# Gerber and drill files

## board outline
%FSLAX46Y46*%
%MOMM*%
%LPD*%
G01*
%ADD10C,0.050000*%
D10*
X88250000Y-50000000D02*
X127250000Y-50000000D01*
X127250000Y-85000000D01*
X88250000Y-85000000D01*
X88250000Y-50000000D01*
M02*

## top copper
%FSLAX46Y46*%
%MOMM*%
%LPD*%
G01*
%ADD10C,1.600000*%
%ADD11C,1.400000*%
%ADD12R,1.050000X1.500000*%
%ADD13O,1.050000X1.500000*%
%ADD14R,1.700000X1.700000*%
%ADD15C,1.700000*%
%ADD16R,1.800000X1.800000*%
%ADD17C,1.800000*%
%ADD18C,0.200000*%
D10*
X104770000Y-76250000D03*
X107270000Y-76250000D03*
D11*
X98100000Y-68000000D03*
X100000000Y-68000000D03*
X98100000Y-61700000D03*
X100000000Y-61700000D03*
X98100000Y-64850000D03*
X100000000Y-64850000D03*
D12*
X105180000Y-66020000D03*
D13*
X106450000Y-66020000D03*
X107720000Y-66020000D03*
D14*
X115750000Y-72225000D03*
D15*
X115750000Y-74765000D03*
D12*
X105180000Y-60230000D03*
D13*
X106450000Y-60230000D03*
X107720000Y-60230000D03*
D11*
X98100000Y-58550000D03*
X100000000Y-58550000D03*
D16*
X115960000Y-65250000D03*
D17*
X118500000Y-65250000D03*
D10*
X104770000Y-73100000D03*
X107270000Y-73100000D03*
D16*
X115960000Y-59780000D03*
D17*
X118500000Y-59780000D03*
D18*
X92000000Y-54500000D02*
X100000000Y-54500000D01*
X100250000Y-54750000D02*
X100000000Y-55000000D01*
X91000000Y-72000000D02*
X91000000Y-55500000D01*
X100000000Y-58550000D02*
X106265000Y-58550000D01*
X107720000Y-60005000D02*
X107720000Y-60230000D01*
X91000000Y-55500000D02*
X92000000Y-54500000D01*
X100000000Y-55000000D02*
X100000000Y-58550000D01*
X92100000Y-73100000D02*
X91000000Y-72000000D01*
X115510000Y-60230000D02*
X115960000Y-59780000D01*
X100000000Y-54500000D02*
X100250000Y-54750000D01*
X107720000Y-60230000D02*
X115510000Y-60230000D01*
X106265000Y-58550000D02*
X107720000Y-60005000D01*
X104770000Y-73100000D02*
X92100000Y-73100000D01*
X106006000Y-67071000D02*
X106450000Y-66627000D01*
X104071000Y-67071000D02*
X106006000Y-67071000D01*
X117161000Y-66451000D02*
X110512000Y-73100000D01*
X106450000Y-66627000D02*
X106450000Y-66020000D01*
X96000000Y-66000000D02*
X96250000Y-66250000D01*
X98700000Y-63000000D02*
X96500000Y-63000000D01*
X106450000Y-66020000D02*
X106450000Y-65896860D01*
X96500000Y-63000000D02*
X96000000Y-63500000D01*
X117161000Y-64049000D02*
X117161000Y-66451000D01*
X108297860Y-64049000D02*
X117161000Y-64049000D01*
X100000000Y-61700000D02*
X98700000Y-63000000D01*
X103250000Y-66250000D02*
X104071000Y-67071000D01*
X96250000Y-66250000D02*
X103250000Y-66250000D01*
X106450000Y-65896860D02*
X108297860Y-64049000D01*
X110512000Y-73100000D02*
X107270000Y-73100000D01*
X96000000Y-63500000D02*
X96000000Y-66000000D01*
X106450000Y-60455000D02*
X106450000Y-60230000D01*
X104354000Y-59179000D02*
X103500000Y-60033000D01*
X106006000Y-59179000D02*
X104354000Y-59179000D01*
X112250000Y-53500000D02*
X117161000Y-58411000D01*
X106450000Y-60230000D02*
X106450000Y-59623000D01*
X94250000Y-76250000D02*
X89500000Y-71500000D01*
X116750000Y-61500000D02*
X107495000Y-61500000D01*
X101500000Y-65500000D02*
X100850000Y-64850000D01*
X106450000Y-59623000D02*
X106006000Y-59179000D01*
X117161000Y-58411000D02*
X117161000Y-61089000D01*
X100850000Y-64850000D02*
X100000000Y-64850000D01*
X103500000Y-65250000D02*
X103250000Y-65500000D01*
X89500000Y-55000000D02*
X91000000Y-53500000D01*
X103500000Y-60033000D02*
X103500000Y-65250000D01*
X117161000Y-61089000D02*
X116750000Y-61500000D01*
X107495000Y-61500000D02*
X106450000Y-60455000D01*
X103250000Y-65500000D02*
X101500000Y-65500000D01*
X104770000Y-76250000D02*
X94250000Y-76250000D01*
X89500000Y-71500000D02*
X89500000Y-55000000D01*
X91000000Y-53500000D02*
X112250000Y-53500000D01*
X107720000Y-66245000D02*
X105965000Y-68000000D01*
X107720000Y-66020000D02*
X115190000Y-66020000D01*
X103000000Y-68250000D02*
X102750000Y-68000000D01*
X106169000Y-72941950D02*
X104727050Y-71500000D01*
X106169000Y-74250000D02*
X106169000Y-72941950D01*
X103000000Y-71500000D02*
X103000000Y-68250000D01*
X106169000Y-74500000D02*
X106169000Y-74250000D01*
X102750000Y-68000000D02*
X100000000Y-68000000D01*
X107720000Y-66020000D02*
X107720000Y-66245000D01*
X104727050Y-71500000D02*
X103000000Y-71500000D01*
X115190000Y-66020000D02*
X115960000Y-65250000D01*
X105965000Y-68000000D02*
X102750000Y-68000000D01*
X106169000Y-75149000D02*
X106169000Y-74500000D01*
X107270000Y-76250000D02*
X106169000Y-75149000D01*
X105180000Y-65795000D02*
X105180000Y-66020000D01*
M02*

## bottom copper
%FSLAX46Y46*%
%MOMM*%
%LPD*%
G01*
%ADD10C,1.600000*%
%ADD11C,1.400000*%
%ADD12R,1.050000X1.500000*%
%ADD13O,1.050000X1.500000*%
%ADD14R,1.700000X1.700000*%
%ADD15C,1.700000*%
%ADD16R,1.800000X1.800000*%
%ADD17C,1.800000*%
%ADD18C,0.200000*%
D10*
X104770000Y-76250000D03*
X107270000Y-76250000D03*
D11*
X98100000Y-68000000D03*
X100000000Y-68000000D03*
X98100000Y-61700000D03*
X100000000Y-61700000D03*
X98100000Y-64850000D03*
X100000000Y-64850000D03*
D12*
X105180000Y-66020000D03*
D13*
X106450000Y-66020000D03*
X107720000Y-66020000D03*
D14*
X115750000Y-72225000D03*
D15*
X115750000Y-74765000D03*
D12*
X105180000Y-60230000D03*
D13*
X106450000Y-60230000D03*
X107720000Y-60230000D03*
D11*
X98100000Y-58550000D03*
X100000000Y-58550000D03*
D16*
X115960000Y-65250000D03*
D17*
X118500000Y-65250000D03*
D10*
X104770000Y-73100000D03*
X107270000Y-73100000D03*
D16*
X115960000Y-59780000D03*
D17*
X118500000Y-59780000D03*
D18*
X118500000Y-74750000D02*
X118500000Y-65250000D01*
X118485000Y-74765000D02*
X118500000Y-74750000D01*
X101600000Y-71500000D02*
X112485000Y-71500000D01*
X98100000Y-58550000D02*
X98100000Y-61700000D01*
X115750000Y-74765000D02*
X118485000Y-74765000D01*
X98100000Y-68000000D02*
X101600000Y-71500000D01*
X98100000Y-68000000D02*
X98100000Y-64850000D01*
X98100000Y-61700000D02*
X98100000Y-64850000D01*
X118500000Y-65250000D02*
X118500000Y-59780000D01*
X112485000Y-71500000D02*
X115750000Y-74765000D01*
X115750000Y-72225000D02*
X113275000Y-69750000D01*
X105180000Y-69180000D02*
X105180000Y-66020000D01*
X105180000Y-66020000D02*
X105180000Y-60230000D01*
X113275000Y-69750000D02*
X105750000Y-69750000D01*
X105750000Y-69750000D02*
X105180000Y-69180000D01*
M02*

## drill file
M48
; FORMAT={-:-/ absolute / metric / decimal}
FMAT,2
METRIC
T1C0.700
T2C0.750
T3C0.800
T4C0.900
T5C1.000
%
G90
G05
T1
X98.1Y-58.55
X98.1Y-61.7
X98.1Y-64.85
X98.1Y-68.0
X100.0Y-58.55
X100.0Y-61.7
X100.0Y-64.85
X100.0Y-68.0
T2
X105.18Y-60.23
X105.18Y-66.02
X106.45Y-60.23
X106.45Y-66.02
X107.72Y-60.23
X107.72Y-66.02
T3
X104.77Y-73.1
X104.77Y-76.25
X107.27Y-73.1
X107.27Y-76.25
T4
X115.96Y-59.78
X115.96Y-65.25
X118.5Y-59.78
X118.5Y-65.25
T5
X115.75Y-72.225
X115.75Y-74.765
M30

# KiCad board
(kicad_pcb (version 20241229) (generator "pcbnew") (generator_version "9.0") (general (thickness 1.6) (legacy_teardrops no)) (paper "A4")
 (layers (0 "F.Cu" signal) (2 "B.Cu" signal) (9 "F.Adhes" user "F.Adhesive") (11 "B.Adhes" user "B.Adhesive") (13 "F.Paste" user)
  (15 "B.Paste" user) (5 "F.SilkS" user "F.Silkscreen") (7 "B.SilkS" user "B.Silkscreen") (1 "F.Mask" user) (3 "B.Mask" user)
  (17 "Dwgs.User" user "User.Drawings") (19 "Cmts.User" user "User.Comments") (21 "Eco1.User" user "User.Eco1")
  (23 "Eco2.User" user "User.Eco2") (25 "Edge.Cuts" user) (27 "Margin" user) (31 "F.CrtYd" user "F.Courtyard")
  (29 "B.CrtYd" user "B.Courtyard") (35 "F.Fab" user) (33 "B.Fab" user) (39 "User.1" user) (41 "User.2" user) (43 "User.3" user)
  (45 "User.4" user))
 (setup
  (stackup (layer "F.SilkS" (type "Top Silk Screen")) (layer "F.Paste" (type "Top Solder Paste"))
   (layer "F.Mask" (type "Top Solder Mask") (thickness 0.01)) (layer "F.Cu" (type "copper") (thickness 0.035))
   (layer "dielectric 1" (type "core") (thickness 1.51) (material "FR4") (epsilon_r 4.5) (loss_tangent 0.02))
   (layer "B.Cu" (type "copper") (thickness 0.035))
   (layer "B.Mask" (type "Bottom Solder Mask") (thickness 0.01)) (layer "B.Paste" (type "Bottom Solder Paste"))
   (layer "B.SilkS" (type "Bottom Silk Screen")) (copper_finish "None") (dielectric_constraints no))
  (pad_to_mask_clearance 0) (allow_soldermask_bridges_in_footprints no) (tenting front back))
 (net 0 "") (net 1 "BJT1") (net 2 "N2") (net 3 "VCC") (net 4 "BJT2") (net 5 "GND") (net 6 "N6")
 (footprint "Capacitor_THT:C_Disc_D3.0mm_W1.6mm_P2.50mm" (layer "F.Cu") (at 104.77 76.25)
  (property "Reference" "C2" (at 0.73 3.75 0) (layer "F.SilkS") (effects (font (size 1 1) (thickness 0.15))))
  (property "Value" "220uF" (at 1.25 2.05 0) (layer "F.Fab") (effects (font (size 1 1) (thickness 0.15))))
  (pad "1" thru_hole circle (at 0 0) (size 1.6 1.6) (drill 0.8) (layers "*.Cu" "*.Mask") (remove_unused_layers no) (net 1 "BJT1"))
  (pad "2" thru_hole circle (at 2.5 0) (size 1.6 1.6) (drill 0.8) (layers "*.Cu" "*.Mask") (remove_unused_layers no) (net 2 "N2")))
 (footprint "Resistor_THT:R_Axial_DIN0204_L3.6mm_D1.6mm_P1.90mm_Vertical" (layer "F.Cu") (at 98.1 68)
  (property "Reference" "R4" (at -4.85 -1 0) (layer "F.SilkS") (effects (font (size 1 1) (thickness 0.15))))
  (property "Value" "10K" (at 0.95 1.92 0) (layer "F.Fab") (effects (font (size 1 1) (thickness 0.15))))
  (pad "1" thru_hole circle (at 0 0) (size 1.4 1.4) (drill 0.7) (layers "*.Cu" "*.Mask") (remove_unused_layers no) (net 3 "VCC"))
  (pad "2" thru_hole circle (at 1.9 0) (size 1.4 1.4) (drill 0.7) (layers "*.Cu" "*.Mask") (remove_unused_layers no) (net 2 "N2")))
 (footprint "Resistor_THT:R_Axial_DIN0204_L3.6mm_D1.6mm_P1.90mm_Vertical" (layer "F.Cu") (at 98.1 61.7)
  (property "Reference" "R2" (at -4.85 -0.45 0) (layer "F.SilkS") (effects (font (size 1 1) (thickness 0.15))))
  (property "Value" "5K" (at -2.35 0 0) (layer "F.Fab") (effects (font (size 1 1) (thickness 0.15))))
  (pad "1" thru_hole circle (at 0 0) (size 1.4 1.4) (drill 0.7) (layers "*.Cu" "*.Mask") (remove_unused_layers no) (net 3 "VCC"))
  (pad "2" thru_hole circle (at 1.9 0) (size 1.4 1.4) (drill 0.7) (layers "*.Cu" "*.Mask") (remove_unused_layers no) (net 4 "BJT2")))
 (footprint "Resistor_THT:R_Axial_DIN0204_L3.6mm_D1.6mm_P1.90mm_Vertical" (layer "F.Cu") (at 98.1 64.85)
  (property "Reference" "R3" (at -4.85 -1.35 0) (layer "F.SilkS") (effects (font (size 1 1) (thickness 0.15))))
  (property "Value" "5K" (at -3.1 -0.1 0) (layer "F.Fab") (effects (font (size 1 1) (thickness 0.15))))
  (pad "1" thru_hole circle (at 0 0) (size 1.4 1.4) (drill 0.7) (layers "*.Cu" "*.Mask") (remove_unused_layers no) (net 3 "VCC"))
  (pad "2" thru_hole circle (at 1.9 0) (size 1.4 1.4) (drill 0.7) (layers "*.Cu" "*.Mask") (remove_unused_layers no) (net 1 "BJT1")))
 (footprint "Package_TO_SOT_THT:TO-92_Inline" (layer "F.Cu") (at 105.18 66.02)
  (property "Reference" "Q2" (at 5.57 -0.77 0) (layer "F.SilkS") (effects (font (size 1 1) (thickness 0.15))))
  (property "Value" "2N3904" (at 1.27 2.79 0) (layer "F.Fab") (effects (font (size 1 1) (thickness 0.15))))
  (pad "1" thru_hole rect (at 0 0) (size 1.05 1.5) (drill 0.75) (layers "*.Cu" "*.Mask") (remove_unused_layers no) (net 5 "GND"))
  (pad "2" thru_hole oval (at 1.27 0) (size 1.05 1.5) (drill 0.75) (layers "*.Cu" "*.Mask") (remove_unused_layers no) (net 4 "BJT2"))
  (pad "3" thru_hole oval (at 2.54 0) (size 1.05 1.5) (drill 0.75) (layers "*.Cu" "*.Mask") (remove_unused_layers no) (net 2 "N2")))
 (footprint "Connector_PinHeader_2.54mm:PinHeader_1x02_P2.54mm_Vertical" (layer "F.Cu") (at 115.75 72.225)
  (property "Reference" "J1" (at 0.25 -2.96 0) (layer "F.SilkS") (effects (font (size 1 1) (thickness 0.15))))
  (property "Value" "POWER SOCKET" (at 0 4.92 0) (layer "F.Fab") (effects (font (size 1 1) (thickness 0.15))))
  (pad "1" thru_hole rect (at 0 0) (size 1.7 1.7) (drill 1) (layers "*.Cu" "*.Mask") (remove_unused_layers no) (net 5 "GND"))
  (pad "2" thru_hole circle (at 0 2.54) (size 1.7 1.7) (drill 1) (layers "*.Cu" "*.Mask") (remove_unused_layers no) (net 3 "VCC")))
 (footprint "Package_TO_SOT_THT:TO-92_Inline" (layer "F.Cu") (at 105.18 60.23)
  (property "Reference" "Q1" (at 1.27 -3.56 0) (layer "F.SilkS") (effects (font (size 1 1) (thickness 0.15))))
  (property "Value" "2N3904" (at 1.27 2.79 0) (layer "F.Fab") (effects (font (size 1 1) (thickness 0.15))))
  (pad "1" thru_hole rect (at 0 0) (size 1.05 1.5) (drill 0.75) (layers "*.Cu" "*.Mask") (remove_unused_layers no) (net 5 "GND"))
  (pad "2" thru_hole oval (at 1.27 0) (size 1.05 1.5) (drill 0.75) (layers "*.Cu" "*.Mask") (remove_unused_layers no) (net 1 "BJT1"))
  (pad "3" thru_hole oval (at 2.54 0) (size 1.05 1.5) (drill 0.75) (layers "*.Cu" "*.Mask") (remove_unused_layers no) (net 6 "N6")))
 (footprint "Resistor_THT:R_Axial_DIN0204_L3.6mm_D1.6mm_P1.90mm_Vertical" (layer "F.Cu") (at 98.1 58.55)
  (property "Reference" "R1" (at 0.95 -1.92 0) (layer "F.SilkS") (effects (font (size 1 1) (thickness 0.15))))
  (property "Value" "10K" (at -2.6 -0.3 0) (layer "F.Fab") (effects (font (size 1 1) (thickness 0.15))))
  (pad "1" thru_hole circle (at 0 0) (size 1.4 1.4) (drill 0.7) (layers "*.Cu" "*.Mask") (remove_unused_layers no) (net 3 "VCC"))
  (pad "2" thru_hole circle (at 1.9 0) (size 1.4 1.4) (drill 0.7) (layers "*.Cu" "*.Mask") (remove_unused_layers no) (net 6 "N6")))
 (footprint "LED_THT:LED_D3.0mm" (layer "F.Cu") (at 115.96 65.25)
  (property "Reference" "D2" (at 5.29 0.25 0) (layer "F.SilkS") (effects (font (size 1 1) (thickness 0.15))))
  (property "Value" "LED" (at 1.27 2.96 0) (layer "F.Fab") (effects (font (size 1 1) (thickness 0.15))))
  (pad "1" thru_hole rect (at 0 0) (size 1.8 1.8) (drill 0.9) (layers "*.Cu" "*.Mask") (remove_unused_layers no) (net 2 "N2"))
  (pad "2" thru_hole circle (at 2.54 0) (size 1.8 1.8) (drill 0.9) (layers "*.Cu" "*.Mask") (remove_unused_layers no) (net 3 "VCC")))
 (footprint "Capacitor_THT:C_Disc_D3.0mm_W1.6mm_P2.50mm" (layer "F.Cu") (at 104.77 73.1)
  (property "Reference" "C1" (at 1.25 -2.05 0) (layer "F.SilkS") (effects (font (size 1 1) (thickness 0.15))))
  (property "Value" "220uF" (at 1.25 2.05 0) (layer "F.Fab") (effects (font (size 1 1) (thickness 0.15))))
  (pad "1" thru_hole circle (at 0 0) (size 1.6 1.6) (drill 0.8) (layers "*.Cu" "*.Mask") (remove_unused_layers no) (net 6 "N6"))
  (pad "2" thru_hole circle (at 2.5 0) (size 1.6 1.6) (drill 0.8) (layers "*.Cu" "*.Mask") (remove_unused_layers no) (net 4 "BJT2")))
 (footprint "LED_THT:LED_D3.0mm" (layer "F.Cu") (at 115.96 59.78)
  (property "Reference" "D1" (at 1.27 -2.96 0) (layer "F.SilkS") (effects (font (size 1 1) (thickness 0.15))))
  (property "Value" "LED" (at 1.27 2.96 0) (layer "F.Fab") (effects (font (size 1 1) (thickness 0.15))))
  (pad "1" thru_hole rect (at 0 0) (size 1.8 1.8) (drill 0.9) (layers "*.Cu" "*.Mask") (remove_unused_layers no) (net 6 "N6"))
  (pad "2" thru_hole circle (at 2.54 0) (size 1.8 1.8) (drill 0.9) (layers "*.Cu" "*.Mask") (remove_unused_layers no) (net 3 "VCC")))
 (gr_rect (start 88.25 50) (end 127.25 85) (stroke (width 0.05) (type default)) (fill no) (layer "Edge.Cuts"))
 (segment (start 118.5 74.75) (end 118.5 65.25) (width 0.2) (layer "B.Cu") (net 3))
 (segment (start 118.485 74.765) (end 118.5 74.75) (width 0.2) (layer "B.Cu") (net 3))
 (segment (start 101.6 71.5) (end 112.485 71.5) (width 0.2) (layer "B.Cu") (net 3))
 (segment (start 98.1 58.55) (end 98.1 61.7) (width 0.2) (layer "B.Cu") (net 3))
 (segment (start 115.75 74.765) (end 118.485 74.765) (width 0.2) (layer "B.Cu") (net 3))
 (segment (start 98.1 68) (end 101.6 71.5) (width 0.2) (layer "B.Cu") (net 3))
 (segment (start 98.1 68) (end 98.1 64.85) (width 0.2) (layer "B.Cu") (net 3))
 (segment (start 98.1 61.7) (end 98.1 64.85) (width 0.2) (layer "B.Cu") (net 3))
 (segment (start 118.5 65.25) (end 118.5 59.78) (width 0.2) (layer "B.Cu") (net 3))
 (segment (start 112.485 71.5) (end 115.75 74.765) (width 0.2) (layer "B.Cu") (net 3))
 (segment (start 92 54.5) (end 100 54.5) (width 0.2) (layer "F.Cu") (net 6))
 (segment (start 100.25 54.75) (end 100 55) (width 0.2) (layer "F.Cu") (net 6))
 (segment (start 91 72) (end 91 55.5) (width 0.2) (layer "F.Cu") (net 6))
 (segment (start 100 58.55) (end 106.265 58.55) (width 0.2) (layer "F.Cu") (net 6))
 (segment (start 107.72 60.005) (end 107.72 60.23) (width 0.2) (layer "F.Cu") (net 6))
 (segment (start 91 55.5) (end 92 54.5) (width 0.2) (layer "F.Cu") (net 6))
 (segment (start 100 55) (end 100 58.55) (width 0.2) (layer "F.Cu") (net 6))
 (segment (start 92.1 73.1) (end 91 72) (width 0.2) (layer "F.Cu") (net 6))
 (segment (start 115.51 60.23) (end 115.96 59.78) (width 0.2) (layer "F.Cu") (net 6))
 (segment (start 100 54.5) (end 100.25 54.75) (width 0.2) (layer "F.Cu") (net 6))
 (segment (start 107.72 60.23) (end 115.51 60.23) (width 0.2) (layer "F.Cu") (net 6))
 (segment (start 106.265 58.55) (end 107.72 60.005) (width 0.2) (layer "F.Cu") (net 6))
 (segment (start 104.77 73.1) (end 92.1 73.1) (width 0.2) (layer "F.Cu") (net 6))
 (segment (start 106.006 67.071) (end 106.45 66.627) (width 0.2) (layer "F.Cu") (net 4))
 (segment (start 104.071 67.071) (end 106.006 67.071) (width 0.2) (layer "F.Cu") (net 4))
 (segment (start 117.161 66.451) (end 110.512 73.1) (width 0.2) (layer "F.Cu") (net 4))
 (segment (start 106.45 66.627) (end 106.45 66.02) (width 0.2) (layer "F.Cu") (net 4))
 (segment (start 96 66) (end 96.25 66.25) (width 0.2) (layer "F.Cu") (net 4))
 (segment (start 98.7 63) (end 96.5 63) (width 0.2) (layer "F.Cu") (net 4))
 (segment (start 106.45 66.02) (end 106.45 65.89686) (width 0.2) (layer "F.Cu") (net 4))
 (segment (start 96.5 63) (end 96 63.5) (width 0.2) (layer "F.Cu") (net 4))
 (segment (start 117.161 64.049) (end 117.161 66.451) (width 0.2) (layer "F.Cu") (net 4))
 (segment (start 108.29786 64.049) (end 117.161 64.049) (width 0.2) (layer "F.Cu") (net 4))
 (segment (start 100 61.7) (end 98.7 63) (width 0.2) (layer "F.Cu") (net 4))
 (segment (start 103.25 66.25) (end 104.071 67.071) (width 0.2) (layer "F.Cu") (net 4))
 (segment (start 96.25 66.25) (end 103.25 66.25) (width 0.2) (layer "F.Cu") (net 4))
 (segment (start 106.45 65.89686) (end 108.29786 64.049) (width 0.2) (layer "F.Cu") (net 4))
 (segment (start 110.512 73.1) (end 107.27 73.1) (width 0.2) (layer "F.Cu") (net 4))
 (segment (start 96 63.5) (end 96 66) (width 0.2) (layer "F.Cu") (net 4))
 (segment (start 106.45 60.455) (end 106.45 60.23) (width 0.2) (layer "F.Cu") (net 1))
 (segment (start 104.354 59.179) (end 103.5 60.033) (width 0.2) (layer "F.Cu") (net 1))
 (segment (start 106.006 59.179) (end 104.354 59.179) (width 0.2) (layer "F.Cu") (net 1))
 (segment (start 112.25 53.5) (end 117.161 58.411) (width 0.2) (layer "F.Cu") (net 1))
 (segment (start 106.45 60.23) (end 106.45 59.623) (width 0.2) (layer "F.Cu") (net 1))
 (segment (start 94.25 76.25) (end 89.5 71.5) (width 0.2) (layer "F.Cu") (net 1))
 (segment (start 116.75 61.5) (end 107.495 61.5) (width 0.2) (layer "F.Cu") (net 1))
 (segment (start 101.5 65.5) (end 100.85 64.85) (width 0.2) (layer "F.Cu") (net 1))
 (segment (start 106.45 59.623) (end 106.006 59.179) (width 0.2) (layer "F.Cu") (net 1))
 (segment (start 117.161 58.411) (end 117.161 61.089) (width 0.2) (layer "F.Cu") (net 1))
 (segment (start 100.85 64.85) (end 100 64.85) (width 0.2) (layer "F.Cu") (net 1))
 (segment (start 103.5 65.25) (end 103.25 65.5) (width 0.2) (layer "F.Cu") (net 1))
 (segment (start 89.5 55) (end 91 53.5) (width 0.2) (layer "F.Cu") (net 1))
 (segment (start 103.5 60.033) (end 103.5 65.25) (width 0.2) (layer "F.Cu") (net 1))
 (segment (start 117.161 61.089) (end 116.75 61.5) (width 0.2) (layer "F.Cu") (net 1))
 (segment (start 107.495 61.5) (end 106.45 60.455) (width 0.2) (layer "F.Cu") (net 1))
 (segment (start 103.25 65.5) (end 101.5 65.5) (width 0.2) (layer "F.Cu") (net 1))
 (segment (start 104.77 76.25) (end 94.25 76.25) (width 0.2) (layer "F.Cu") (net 1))
 (segment (start 89.5 71.5) (end 89.5 55) (width 0.2) (layer "F.Cu") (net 1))
 (segment (start 91 53.5) (end 112.25 53.5) (width 0.2) (layer "F.Cu") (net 1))
 (segment (start 107.72 66.245) (end 105.965 68) (width 0.2) (layer "F.Cu") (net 2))
 (segment (start 107.72 66.02) (end 115.19 66.02) (width 0.2) (layer "F.Cu") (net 2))
 (segment (start 103 68.25) (end 102.75 68) (width 0.2) (layer "F.Cu") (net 2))
 (segment (start 106.169 72.94195) (end 104.72705 71.5) (width 0.2) (layer "F.Cu") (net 2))
 (segment (start 106.169 74.25) (end 106.169 72.94195) (width 0.2) (layer "F.Cu") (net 2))
 (segment (start 103 71.5) (end 103 68.25) (width 0.2) (layer "F.Cu") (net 2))
 (segment (start 106.169 74.5) (end 106.169 74.25) (width 0.2) (layer "F.Cu") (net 2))
 (segment (start 102.75 68) (end 100 68) (width 0.2) (layer "F.Cu") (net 2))
 (segment (start 107.72 66.02) (end 107.72 66.245) (width 0.2) (layer "F.Cu") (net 2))
 (segment (start 104.72705 71.5) (end 103 71.5) (width 0.2) (layer "F.Cu") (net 2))
 (segment (start 115.19 66.02) (end 115.96 65.25) (width 0.2) (layer "F.Cu") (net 2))
 (segment (start 105.965 68) (end 102.75 68) (width 0.2) (layer "F.Cu") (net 2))
 (segment (start 106.169 75.149) (end 106.169 74.5) (width 0.2) (layer "F.Cu") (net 2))
 (segment (start 107.27 76.25) (end 106.169 75.149) (width 0.2) (layer "F.Cu") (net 2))
 (segment (start 105.18 65.795) (end 105.18 66.02) (width 0.2) (layer "F.Cu") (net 5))
 (segment (start 115.75 72.225) (end 113.275 69.75) (width 0.2) (layer "B.Cu") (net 5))
 (segment (start 105.18 69.18) (end 105.18 66.02) (width 0.2) (layer "B.Cu") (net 5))
 (segment (start 105.18 66.02) (end 105.18 60.23) (width 0.2) (layer "B.Cu") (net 5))
 (segment (start 113.275 69.75) (end 105.75 69.75) (width 0.2) (layer "B.Cu") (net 5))
 (segment (start 105.75 69.75) (end 105.18 69.18) (width 0.2) (layer "B.Cu") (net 5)))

